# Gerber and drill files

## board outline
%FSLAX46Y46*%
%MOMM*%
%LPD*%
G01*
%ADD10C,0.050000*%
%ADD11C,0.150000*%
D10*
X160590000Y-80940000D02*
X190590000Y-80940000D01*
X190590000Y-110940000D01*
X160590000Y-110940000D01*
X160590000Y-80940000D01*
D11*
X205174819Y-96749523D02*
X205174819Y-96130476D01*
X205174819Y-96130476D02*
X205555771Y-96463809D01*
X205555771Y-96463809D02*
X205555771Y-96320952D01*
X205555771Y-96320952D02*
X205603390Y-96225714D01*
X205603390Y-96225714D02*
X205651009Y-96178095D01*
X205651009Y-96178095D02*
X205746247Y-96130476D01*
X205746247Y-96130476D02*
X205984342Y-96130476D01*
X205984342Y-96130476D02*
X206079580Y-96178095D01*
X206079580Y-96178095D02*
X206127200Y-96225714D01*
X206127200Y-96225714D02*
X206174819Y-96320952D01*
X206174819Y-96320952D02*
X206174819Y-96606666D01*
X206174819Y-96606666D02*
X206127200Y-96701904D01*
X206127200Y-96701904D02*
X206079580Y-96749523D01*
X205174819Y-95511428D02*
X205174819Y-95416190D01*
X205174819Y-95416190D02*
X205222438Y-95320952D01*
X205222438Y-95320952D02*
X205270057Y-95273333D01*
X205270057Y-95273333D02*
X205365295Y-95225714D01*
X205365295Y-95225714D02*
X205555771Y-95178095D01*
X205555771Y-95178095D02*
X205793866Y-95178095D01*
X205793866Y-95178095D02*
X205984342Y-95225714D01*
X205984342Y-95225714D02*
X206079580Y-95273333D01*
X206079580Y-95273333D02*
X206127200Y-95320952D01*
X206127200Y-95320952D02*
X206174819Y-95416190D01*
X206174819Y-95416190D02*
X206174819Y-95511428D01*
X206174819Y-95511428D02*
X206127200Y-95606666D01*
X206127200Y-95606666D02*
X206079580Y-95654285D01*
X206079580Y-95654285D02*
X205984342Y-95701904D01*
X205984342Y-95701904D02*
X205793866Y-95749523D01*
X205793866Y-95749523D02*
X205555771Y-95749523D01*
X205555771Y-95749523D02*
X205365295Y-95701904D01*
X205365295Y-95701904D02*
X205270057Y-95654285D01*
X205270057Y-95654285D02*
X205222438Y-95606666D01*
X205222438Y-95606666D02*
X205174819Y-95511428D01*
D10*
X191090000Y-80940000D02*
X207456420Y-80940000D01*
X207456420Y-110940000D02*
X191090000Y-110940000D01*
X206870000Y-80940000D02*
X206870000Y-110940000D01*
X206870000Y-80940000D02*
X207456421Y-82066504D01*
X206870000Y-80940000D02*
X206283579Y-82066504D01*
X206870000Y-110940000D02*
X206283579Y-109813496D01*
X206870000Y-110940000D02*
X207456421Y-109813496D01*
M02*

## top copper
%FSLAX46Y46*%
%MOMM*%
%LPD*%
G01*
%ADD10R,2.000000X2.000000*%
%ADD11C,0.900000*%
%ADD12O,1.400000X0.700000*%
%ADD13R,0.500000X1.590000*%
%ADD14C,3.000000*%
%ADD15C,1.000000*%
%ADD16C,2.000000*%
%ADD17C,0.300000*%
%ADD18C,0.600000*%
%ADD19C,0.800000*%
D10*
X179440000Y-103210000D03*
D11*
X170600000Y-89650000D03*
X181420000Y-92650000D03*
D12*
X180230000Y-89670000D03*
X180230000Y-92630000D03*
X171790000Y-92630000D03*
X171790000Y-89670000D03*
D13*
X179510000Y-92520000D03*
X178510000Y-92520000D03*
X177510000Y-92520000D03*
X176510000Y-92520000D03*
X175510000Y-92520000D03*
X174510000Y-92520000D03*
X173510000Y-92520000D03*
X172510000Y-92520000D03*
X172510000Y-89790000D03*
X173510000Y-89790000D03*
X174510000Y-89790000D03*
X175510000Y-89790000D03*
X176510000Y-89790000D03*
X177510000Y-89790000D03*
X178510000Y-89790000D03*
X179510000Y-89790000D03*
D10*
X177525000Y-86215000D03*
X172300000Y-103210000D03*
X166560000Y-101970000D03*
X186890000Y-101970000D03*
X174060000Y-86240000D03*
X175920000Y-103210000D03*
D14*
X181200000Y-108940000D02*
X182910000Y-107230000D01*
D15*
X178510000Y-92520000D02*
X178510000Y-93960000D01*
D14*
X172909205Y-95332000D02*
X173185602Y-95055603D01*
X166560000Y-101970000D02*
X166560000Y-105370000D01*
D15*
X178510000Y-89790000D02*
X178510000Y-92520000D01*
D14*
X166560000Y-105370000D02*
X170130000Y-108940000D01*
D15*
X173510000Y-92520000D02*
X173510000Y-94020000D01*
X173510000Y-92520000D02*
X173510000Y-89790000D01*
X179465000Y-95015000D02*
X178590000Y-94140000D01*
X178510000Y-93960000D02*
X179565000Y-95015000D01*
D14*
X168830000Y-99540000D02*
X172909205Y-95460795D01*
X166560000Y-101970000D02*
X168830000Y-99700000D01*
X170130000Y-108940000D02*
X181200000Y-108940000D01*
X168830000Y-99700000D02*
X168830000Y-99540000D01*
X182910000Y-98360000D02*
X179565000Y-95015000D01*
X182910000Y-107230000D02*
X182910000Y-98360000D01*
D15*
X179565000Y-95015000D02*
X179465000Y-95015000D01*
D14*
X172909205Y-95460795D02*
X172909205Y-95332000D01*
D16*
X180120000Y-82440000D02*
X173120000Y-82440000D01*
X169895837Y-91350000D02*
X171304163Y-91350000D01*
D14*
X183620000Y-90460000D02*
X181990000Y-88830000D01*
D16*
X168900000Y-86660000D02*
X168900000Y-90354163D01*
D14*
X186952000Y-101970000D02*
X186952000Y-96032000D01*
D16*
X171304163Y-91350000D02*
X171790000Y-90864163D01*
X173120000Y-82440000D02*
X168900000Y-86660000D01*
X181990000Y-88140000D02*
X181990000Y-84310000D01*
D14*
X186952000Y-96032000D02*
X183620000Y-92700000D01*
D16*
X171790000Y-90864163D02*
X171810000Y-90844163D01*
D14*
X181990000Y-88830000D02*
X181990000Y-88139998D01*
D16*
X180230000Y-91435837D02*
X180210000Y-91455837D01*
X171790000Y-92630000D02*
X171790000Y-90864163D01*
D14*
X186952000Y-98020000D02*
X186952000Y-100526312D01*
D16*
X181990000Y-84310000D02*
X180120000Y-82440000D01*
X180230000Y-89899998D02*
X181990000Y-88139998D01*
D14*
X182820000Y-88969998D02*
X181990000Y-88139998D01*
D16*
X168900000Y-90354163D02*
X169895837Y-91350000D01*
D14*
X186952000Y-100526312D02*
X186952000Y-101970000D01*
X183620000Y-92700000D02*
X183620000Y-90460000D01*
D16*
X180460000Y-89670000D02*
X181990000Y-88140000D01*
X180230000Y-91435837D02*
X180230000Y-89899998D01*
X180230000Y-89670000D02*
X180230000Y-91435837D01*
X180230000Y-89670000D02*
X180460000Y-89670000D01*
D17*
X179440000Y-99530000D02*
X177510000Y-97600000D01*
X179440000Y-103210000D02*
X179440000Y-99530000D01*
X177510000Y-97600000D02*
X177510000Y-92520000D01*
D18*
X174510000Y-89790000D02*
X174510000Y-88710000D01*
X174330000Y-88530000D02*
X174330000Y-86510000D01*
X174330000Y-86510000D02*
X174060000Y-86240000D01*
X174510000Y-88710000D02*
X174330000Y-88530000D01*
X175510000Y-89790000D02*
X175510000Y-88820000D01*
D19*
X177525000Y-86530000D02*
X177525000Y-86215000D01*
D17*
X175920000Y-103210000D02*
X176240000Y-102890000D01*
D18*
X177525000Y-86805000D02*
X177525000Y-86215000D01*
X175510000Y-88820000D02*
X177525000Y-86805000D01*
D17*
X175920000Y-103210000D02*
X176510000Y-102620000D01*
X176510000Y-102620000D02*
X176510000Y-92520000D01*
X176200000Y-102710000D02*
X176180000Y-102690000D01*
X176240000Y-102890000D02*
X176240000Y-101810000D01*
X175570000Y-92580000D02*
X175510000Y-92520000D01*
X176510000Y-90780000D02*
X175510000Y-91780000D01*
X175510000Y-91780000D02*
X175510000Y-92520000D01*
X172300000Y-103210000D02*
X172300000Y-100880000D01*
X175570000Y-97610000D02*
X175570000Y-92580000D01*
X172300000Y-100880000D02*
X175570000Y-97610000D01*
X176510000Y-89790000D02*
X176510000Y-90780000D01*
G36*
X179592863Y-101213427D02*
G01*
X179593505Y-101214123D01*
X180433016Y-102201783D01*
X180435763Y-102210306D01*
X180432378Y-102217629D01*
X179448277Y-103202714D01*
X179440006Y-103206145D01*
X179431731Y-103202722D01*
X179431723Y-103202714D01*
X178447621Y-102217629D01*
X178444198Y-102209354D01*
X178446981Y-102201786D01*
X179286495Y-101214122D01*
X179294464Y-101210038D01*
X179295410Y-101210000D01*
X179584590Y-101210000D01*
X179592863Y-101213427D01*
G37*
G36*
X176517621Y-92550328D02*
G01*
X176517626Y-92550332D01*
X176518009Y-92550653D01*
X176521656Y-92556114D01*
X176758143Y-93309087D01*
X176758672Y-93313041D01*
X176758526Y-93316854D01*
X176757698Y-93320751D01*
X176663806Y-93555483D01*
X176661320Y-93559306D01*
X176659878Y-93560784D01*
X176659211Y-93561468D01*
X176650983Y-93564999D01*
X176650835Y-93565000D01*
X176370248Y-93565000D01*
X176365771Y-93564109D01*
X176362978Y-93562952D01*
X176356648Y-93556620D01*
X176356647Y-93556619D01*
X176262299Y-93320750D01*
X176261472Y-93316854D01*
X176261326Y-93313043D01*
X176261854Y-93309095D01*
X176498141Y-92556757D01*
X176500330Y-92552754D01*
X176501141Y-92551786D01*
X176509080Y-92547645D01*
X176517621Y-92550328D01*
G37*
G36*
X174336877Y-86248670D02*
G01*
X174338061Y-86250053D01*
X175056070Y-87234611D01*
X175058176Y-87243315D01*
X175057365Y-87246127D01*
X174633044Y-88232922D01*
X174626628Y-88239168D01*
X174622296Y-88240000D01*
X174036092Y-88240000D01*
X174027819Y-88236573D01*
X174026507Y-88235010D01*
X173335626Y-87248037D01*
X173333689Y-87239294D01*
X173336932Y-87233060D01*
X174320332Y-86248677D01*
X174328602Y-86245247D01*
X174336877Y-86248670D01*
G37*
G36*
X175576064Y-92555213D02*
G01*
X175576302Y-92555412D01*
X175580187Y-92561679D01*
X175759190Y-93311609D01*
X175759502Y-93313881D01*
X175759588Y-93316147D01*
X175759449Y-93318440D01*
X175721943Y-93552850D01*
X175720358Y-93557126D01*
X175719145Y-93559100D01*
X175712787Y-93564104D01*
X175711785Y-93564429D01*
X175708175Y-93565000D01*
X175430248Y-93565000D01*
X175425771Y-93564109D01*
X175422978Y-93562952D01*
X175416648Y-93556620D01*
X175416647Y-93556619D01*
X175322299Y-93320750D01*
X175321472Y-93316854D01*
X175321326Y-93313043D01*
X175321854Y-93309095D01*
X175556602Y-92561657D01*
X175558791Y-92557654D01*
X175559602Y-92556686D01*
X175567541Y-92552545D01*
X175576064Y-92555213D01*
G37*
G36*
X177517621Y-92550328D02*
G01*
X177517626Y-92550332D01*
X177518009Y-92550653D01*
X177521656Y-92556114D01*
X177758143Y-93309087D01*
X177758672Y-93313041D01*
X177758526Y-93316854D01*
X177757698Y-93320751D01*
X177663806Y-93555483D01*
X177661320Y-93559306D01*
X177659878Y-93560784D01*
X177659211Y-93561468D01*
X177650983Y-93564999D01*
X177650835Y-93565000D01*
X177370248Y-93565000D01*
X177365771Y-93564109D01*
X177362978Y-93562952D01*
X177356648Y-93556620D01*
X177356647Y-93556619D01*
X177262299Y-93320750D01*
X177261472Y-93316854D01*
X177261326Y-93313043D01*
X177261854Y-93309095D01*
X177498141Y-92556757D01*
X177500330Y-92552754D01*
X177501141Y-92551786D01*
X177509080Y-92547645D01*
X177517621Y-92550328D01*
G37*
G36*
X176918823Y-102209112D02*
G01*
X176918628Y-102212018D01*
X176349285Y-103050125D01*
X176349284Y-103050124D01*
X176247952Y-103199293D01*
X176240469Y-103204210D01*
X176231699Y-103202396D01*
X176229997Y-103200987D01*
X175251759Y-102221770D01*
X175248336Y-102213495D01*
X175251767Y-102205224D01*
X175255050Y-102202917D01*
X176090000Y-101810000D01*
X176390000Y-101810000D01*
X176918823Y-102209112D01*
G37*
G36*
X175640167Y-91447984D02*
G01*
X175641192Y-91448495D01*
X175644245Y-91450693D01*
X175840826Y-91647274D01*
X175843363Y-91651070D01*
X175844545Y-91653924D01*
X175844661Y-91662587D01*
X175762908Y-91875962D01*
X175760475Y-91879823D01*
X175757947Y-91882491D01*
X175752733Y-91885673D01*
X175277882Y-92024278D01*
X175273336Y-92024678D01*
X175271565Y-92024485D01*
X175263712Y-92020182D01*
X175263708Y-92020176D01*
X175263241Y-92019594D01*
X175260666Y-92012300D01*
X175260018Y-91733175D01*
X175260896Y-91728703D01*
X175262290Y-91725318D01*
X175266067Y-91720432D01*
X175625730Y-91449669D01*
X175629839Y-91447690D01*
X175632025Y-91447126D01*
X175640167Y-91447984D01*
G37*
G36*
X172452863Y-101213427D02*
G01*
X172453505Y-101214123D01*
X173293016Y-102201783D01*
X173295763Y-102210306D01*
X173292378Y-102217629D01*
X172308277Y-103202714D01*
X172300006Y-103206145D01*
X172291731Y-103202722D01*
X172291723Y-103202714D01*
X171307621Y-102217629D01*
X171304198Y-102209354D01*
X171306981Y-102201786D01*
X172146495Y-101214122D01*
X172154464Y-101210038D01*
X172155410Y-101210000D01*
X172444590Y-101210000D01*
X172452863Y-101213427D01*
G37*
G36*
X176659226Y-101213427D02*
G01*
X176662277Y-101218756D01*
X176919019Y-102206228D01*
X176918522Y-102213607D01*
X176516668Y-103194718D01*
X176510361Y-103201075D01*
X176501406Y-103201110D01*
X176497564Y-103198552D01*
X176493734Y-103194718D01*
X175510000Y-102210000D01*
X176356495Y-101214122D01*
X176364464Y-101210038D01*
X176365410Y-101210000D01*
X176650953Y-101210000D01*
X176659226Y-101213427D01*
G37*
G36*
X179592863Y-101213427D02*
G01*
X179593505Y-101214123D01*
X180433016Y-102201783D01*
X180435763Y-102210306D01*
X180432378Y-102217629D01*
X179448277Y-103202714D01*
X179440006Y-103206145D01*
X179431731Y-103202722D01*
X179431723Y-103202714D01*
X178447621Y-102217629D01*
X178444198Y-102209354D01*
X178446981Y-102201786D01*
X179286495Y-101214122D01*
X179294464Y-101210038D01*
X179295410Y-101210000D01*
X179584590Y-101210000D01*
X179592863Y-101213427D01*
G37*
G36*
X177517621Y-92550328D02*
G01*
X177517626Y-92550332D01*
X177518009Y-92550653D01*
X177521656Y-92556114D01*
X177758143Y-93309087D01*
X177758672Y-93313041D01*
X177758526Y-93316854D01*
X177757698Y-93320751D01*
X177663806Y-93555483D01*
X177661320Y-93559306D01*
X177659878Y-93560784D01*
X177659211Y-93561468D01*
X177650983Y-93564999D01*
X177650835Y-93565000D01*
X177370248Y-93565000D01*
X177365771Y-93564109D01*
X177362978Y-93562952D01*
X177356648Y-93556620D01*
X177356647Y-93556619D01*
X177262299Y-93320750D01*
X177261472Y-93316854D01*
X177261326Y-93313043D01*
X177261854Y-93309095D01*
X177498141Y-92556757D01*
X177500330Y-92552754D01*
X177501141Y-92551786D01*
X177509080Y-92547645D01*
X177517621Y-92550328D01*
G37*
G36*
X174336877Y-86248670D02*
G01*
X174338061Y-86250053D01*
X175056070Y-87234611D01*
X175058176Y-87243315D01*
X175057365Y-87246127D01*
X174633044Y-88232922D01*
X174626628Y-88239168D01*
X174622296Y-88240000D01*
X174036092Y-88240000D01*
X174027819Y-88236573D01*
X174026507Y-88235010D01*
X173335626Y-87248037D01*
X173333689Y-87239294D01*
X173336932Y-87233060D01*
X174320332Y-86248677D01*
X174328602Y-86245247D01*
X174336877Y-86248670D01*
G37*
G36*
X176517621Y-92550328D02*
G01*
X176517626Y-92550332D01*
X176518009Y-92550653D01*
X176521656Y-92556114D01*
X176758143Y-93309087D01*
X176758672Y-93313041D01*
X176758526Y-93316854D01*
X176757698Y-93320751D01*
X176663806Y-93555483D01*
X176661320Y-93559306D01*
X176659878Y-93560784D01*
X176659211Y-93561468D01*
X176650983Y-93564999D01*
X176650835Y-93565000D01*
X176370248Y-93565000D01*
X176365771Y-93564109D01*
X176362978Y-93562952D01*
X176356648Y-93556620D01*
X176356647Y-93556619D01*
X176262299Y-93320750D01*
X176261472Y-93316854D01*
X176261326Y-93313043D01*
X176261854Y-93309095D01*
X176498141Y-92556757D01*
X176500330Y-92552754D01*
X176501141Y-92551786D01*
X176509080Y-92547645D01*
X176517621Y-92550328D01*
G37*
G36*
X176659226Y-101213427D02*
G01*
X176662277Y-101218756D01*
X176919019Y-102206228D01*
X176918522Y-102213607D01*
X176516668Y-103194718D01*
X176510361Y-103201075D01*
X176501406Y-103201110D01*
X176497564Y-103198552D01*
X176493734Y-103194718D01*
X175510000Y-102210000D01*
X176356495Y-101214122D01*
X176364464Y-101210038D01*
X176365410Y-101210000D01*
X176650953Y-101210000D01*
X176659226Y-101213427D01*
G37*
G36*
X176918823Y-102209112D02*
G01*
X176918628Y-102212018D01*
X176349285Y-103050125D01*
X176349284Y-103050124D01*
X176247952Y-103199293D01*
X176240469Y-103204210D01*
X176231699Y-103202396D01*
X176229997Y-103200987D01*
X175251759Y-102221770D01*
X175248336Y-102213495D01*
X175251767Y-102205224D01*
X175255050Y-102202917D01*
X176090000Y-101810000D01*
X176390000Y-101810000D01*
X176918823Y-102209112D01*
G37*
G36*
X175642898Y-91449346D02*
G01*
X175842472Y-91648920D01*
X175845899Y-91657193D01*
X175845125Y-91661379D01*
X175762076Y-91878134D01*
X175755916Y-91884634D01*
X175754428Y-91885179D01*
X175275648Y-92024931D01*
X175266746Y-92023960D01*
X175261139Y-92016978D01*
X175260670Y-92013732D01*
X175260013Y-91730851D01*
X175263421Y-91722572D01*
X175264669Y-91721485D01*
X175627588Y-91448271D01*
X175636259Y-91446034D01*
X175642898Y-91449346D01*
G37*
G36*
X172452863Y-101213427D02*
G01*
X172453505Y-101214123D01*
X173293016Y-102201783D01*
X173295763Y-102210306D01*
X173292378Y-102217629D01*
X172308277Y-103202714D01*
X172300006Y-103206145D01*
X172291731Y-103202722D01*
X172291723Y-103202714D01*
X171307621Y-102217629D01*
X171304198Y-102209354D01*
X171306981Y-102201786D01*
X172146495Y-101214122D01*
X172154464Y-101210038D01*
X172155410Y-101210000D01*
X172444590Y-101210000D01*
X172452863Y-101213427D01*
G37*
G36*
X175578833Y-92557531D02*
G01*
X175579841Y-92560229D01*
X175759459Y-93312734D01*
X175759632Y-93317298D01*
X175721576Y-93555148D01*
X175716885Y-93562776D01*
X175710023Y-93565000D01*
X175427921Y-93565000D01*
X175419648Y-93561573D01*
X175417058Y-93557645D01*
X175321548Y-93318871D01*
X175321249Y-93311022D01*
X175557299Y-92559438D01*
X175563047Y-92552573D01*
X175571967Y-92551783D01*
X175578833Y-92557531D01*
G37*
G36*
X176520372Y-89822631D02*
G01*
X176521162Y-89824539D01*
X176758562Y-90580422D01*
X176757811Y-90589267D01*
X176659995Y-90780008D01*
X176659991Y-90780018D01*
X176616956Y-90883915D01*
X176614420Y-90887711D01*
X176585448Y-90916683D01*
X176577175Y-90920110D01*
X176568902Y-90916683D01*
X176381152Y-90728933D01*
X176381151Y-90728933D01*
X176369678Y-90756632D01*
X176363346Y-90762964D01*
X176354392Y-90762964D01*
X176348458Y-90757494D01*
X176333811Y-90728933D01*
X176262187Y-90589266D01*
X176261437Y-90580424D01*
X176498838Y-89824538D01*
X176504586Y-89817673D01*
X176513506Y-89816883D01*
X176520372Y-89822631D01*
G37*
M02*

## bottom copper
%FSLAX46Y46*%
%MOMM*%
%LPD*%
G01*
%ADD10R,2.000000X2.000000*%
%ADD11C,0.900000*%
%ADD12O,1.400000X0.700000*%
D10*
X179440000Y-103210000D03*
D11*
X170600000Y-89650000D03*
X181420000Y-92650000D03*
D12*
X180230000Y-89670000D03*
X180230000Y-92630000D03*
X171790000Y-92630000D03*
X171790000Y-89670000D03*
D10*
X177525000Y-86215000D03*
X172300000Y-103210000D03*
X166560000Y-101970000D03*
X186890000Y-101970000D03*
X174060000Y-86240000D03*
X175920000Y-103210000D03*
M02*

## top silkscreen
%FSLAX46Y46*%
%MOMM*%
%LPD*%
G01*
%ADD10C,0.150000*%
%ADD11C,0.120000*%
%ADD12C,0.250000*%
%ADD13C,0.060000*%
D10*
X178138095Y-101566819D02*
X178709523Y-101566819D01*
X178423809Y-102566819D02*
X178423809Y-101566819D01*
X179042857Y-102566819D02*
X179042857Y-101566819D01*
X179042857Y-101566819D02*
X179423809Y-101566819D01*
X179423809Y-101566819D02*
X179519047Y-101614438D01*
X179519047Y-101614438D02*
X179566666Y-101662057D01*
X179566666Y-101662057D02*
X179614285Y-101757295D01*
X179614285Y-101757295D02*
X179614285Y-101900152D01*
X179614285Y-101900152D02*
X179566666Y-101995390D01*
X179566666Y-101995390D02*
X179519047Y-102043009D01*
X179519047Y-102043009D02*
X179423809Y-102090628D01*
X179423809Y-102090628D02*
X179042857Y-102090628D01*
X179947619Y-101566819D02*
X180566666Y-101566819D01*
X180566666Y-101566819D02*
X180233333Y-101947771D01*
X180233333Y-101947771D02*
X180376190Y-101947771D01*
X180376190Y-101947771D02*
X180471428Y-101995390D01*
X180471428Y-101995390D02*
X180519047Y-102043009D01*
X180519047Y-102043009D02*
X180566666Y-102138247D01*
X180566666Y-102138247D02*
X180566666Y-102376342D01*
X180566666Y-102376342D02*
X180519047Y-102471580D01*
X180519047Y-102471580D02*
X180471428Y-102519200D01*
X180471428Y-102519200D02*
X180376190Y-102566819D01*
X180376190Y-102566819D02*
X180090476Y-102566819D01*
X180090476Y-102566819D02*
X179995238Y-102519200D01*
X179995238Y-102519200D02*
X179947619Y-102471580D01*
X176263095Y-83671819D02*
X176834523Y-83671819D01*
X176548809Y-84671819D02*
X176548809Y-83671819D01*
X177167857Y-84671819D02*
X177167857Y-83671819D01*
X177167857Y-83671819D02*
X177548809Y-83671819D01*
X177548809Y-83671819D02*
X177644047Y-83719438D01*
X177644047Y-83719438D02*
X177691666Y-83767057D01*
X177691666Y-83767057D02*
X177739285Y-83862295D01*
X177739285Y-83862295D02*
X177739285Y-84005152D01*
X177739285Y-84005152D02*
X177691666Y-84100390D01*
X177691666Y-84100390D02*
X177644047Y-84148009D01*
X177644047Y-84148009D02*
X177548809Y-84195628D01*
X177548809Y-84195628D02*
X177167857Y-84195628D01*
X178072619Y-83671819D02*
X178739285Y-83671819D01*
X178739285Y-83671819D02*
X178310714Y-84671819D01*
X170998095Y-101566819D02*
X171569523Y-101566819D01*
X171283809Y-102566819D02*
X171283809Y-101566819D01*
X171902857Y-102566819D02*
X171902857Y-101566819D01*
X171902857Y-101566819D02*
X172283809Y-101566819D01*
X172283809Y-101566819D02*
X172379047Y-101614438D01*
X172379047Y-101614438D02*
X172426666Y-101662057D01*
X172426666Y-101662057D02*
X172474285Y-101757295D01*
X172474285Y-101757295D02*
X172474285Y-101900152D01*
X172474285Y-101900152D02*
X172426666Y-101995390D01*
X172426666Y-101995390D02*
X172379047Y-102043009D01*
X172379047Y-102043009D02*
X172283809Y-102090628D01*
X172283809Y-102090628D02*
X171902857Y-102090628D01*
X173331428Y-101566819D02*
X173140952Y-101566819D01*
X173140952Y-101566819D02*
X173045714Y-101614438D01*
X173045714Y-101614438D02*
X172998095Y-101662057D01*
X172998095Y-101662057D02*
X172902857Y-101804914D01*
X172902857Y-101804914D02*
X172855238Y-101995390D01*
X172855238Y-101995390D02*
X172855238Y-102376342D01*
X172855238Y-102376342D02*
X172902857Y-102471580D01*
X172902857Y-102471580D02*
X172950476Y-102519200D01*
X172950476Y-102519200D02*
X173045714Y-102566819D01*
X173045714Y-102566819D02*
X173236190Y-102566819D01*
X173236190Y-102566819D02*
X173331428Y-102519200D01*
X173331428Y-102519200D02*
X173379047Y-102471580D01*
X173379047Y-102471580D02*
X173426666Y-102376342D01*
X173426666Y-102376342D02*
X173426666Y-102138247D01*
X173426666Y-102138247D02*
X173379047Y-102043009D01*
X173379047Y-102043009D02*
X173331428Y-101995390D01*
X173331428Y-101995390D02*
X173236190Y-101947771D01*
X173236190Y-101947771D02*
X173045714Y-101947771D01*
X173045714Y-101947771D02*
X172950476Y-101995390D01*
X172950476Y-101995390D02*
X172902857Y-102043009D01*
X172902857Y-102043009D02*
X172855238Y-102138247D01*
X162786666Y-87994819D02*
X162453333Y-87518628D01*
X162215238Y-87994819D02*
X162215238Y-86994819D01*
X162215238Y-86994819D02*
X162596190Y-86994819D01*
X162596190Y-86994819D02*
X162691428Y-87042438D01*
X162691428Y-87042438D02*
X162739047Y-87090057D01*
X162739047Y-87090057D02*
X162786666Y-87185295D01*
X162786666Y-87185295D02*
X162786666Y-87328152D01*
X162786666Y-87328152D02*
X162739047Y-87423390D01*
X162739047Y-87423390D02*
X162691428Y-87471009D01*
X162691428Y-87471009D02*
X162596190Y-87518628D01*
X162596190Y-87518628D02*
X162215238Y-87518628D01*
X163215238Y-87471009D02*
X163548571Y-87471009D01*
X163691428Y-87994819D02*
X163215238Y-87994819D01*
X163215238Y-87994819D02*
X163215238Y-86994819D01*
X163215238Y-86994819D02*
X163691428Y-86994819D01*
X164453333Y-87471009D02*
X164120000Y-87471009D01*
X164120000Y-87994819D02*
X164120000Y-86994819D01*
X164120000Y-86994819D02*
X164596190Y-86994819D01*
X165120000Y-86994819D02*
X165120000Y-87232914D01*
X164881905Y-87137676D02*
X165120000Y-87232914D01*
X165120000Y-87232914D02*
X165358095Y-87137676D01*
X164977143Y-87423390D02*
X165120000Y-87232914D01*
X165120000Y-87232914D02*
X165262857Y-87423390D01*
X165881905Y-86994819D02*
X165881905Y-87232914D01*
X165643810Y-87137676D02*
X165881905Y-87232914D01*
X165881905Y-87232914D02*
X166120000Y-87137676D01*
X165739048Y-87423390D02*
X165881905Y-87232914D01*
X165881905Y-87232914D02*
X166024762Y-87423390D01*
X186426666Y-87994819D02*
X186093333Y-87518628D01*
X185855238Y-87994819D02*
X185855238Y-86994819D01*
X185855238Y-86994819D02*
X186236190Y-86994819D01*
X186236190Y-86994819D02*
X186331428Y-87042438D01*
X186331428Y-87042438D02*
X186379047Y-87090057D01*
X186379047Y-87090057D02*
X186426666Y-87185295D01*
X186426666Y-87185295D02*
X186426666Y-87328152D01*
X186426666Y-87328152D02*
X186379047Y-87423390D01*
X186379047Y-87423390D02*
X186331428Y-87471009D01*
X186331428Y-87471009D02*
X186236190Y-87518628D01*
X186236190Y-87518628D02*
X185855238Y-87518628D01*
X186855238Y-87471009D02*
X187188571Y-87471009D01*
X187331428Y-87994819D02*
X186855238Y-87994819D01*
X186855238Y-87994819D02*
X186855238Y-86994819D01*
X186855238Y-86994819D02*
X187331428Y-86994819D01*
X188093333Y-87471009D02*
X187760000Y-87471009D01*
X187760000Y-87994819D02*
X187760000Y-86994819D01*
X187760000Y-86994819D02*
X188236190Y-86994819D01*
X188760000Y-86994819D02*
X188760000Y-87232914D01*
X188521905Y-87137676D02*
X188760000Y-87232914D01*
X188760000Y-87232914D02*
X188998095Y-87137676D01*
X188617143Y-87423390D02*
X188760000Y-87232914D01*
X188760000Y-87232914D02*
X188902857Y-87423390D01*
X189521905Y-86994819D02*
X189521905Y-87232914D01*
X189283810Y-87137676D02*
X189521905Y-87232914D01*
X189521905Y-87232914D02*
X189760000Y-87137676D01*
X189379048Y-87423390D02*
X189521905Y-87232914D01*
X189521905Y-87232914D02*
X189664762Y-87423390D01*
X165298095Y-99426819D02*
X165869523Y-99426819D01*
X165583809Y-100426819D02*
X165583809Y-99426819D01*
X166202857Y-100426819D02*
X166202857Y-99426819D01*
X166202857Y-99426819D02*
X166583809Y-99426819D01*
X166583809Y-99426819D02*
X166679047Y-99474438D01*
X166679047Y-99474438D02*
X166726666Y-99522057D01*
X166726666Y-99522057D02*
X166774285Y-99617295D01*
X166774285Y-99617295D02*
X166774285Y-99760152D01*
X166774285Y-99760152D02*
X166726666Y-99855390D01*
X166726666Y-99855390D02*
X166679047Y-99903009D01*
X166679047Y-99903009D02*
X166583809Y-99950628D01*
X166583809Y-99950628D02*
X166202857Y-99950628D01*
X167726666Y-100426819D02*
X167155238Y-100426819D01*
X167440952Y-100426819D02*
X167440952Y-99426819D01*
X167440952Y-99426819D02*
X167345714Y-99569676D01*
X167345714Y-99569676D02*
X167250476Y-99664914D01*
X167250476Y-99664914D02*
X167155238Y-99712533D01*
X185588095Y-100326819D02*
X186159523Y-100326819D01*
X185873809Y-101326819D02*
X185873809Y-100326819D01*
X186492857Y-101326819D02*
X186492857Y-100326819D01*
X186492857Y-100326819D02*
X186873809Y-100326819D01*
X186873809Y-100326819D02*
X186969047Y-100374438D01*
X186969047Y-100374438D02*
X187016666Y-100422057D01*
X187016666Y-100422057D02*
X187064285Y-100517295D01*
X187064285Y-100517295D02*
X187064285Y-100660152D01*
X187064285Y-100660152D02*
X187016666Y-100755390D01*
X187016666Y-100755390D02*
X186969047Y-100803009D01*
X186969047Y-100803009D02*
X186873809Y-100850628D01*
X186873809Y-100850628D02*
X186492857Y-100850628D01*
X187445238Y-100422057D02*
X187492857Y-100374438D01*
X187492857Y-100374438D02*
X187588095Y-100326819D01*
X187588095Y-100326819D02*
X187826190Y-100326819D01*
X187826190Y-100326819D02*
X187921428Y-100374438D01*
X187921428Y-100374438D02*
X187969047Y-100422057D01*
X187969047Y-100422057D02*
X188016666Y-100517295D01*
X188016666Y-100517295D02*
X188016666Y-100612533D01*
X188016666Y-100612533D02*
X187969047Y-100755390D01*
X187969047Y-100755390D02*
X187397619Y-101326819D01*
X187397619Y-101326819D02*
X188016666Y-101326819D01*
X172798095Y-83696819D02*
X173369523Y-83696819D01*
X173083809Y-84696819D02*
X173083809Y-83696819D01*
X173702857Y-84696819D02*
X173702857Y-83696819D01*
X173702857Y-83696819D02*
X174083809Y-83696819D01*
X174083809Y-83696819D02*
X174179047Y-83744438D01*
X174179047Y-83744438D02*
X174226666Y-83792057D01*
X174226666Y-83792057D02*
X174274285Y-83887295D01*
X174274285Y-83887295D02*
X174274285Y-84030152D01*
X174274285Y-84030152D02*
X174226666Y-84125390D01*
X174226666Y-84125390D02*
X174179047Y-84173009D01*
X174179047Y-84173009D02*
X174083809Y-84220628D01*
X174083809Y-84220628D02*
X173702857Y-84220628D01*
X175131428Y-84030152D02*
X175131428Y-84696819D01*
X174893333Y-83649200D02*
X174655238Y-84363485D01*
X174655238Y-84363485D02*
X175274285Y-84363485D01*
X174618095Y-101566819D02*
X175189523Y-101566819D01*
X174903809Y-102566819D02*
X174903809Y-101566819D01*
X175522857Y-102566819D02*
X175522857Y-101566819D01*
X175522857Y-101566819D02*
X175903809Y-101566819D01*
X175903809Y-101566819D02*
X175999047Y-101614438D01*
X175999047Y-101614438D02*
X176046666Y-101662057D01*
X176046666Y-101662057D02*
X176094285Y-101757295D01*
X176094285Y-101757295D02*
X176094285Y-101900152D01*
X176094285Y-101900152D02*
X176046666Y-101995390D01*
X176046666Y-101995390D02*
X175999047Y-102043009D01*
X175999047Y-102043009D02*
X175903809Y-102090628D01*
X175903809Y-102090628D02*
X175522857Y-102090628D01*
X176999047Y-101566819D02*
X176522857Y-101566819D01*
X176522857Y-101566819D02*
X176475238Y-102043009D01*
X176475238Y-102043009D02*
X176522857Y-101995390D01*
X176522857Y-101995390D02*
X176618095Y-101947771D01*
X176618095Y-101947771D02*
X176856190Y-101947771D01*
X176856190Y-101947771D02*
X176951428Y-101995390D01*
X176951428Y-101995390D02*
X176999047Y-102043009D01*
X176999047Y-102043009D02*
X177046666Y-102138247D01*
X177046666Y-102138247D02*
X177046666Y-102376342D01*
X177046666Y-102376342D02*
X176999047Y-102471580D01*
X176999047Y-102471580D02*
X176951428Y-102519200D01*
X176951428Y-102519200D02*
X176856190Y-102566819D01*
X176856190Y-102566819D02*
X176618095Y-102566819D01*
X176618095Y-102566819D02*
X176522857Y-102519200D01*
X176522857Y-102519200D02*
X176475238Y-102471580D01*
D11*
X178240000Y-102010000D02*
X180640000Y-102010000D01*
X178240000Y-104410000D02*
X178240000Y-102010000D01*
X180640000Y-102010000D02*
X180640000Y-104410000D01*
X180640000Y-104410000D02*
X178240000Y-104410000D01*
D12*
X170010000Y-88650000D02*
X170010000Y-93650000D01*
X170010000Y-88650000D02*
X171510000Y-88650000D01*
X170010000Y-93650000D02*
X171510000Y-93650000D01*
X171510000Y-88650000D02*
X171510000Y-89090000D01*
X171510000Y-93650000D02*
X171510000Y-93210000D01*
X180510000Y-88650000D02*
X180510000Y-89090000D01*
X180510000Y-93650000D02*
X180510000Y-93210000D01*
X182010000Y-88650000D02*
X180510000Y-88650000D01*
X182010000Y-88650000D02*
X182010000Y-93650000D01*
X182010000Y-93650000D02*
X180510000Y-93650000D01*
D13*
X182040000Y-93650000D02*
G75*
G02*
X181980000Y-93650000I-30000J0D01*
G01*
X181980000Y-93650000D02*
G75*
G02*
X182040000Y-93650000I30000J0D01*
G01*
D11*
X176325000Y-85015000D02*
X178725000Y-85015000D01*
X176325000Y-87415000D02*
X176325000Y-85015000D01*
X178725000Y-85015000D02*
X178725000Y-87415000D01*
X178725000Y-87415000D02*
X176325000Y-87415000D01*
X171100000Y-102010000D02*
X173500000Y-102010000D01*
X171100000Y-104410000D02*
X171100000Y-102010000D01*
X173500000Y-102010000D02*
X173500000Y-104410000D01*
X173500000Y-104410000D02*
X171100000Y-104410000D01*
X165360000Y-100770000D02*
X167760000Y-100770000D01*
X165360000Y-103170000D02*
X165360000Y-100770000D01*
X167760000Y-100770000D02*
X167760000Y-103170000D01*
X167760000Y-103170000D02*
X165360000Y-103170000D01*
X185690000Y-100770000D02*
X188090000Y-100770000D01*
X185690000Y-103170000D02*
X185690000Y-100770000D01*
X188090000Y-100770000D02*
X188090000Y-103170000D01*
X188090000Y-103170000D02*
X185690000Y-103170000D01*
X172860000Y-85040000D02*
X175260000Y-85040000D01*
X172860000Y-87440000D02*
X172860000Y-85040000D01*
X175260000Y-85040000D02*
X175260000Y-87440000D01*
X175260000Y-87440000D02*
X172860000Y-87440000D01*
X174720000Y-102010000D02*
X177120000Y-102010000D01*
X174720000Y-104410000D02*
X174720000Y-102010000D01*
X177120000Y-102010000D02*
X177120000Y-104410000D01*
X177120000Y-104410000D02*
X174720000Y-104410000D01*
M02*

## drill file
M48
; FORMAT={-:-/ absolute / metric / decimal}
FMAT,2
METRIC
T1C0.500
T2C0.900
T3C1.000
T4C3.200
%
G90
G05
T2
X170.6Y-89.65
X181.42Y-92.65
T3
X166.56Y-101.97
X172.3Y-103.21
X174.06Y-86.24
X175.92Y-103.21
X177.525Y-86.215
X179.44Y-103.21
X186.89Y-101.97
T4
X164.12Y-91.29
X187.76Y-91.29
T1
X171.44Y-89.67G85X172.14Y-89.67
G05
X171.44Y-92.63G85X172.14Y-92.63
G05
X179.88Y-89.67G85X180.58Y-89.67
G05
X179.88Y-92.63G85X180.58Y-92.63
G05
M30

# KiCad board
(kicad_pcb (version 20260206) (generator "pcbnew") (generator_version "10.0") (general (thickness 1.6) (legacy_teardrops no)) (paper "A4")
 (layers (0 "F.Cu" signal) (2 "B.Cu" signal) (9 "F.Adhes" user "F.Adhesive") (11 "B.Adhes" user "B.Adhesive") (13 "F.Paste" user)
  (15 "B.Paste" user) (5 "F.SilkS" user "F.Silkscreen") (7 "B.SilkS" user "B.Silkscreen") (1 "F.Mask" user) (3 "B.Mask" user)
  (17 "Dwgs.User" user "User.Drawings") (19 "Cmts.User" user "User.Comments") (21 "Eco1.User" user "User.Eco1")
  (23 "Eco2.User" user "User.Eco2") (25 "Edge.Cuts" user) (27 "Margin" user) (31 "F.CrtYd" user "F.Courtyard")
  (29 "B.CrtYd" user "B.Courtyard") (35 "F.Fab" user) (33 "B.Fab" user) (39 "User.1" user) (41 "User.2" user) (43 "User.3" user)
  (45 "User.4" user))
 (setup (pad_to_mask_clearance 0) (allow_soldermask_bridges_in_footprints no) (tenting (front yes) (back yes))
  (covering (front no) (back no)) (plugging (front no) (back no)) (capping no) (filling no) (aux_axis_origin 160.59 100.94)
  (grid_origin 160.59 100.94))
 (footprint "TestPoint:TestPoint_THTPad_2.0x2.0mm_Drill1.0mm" (layer "F.Cu") (at 179.44 103.21)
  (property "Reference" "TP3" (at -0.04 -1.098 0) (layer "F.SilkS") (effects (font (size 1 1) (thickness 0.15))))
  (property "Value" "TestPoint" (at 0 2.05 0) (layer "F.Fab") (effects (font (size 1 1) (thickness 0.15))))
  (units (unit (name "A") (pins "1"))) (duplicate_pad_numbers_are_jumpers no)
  (fp_line (start -1.2 -1.2) (end 1.2 -1.2) (stroke (width 0.12) (type solid)) (layer "F.SilkS"))
  (fp_line (start -1.2 1.2) (end -1.2 -1.2) (stroke (width 0.12) (type solid)) (layer "F.SilkS"))
  (fp_line (start 1.2 -1.2) (end 1.2 1.2) (stroke (width 0.12) (type solid)) (layer "F.SilkS"))
  (fp_line (start 1.2 1.2) (end -1.2 1.2) (stroke (width 0.12) (type solid)) (layer "F.SilkS"))
  (pad "1" thru_hole rect (at 0 0) (size 2 2) (drill 1) (layers "*.Cu" "*.Mask") (remove_unused_layers no) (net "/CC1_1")
   (teardrops (best_length_ratio 0.5) (max_length 1) (best_width_ratio 1) (max_width 2) (curved_edges no) (filter_ratio 0.9) (enabled yes)
    (allow_two_segments yes) (prefer_zone_connections yes))))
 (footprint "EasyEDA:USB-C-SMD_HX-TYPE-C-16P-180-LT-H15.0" (layer "F.Cu") (at 176.01 91.15)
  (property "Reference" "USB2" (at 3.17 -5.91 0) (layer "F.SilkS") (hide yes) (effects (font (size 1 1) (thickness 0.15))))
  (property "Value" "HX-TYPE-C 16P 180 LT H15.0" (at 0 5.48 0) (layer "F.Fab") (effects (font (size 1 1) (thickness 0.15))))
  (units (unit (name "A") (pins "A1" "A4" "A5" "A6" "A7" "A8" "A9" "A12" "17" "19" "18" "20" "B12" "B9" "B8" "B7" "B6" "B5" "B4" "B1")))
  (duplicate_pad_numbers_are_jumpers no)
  (fp_line (start -6 -2.5) (end -6 2.5) (stroke (width 0.25) (type solid)) (layer "F.SilkS"))
  (fp_line (start -6 -2.5) (end -4.5 -2.5) (stroke (width 0.25) (type solid)) (layer "F.SilkS"))
  (fp_line (start -6 2.5) (end -4.5 2.5) (stroke (width 0.25) (type solid)) (layer "F.SilkS"))
  (fp_line (start -4.5 -2.5) (end -4.5 -2.06) (stroke (width 0.25) (type solid)) (layer "F.SilkS"))
  (fp_line (start -4.5 2.5) (end -4.5 2.06) (stroke (width 0.25) (type solid)) (layer "F.SilkS"))
  (fp_line (start 4.5 -2.5) (end 4.5 -2.06) (stroke (width 0.25) (type solid)) (layer "F.SilkS"))
  (fp_line (start 4.5 2.5) (end 4.5 2.06) (stroke (width 0.25) (type solid)) (layer "F.SilkS"))
  (fp_line (start 6 -2.5) (end 4.5 -2.5) (stroke (width 0.25) (type solid)) (layer "F.SilkS"))
  (fp_line (start 6 -2.5) (end 6 2.5) (stroke (width 0.25) (type solid)) (layer "F.SilkS"))
  (fp_line (start 6 2.5) (end 4.5 2.5) (stroke (width 0.25) (type solid)) (layer "F.SilkS"))
  (fp_circle (center 6 2.5) (end 6.03 2.5) (stroke (width 0.06) (type solid)) (fill no) (layer "F.SilkS"))
  (pad "" thru_hole circle (at -5.41 -1.5) (size 0.9 0.9) (drill 0.9) (layers "*.Cu" "*.Mask") (remove_unused_layers no)
   (teardrops (best_length_ratio 0.5) (max_length 1) (best_width_ratio 1) (max_width 2) (curved_edges no) (filter_ratio 0.9) (enabled yes)
    (allow_two_segments yes) (prefer_zone_connections yes)))
  (pad "" thru_hole circle (at 5.41 1.5) (size 0.9 0.9) (drill 0.9) (layers "*.Cu" "*.Mask") (remove_unused_layers no)
   (teardrops (best_length_ratio 0.5) (max_length 1) (best_width_ratio 1) (max_width 2) (curved_edges no) (filter_ratio 0.9) (enabled yes)
    (allow_two_segments yes) (prefer_zone_connections yes)))
  (pad "17" thru_hole oval (at 4.22 -1.48 90) (size 0.7 1.4) (drill oval 0.500024 1.199998) (layers "*.Cu" "*.Mask")
   (remove_unused_layers no) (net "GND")
   (teardrops (best_length_ratio 0.5) (max_length 1) (best_width_ratio 1) (max_width 2) (curved_edges no) (filter_ratio 0.9) (enabled yes)
    (allow_two_segments yes) (prefer_zone_connections yes)))
  (pad "18" thru_hole oval (at 4.22 1.48 90) (size 0.7 1.4) (drill oval 0.500024 1.199998) (layers "*.Cu" "*.Mask")
   (remove_unused_layers no) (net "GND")
   (teardrops (best_length_ratio 0.5) (max_length 1) (best_width_ratio 1) (max_width 2) (curved_edges no) (filter_ratio 0.9) (enabled yes)
    (allow_two_segments yes) (prefer_zone_connections yes)))
  (pad "19" thru_hole oval (at -4.22 1.48 90) (size 0.7 1.4) (drill oval 0.500024 1.199998) (layers "*.Cu" "*.Mask")
   (remove_unused_layers no) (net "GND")
   (teardrops (best_length_ratio 0.5) (max_length 1) (best_width_ratio 1) (max_width 2) (curved_edges no) (filter_ratio 0.9) (enabled yes)
    (allow_two_segments yes) (prefer_zone_connections yes)))
  (pad "20" thru_hole oval (at -4.22 -1.48 90) (size 0.7 1.4) (drill oval 0.500024 1.199998) (layers "*.Cu" "*.Mask")
   (remove_unused_layers no) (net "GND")
   (teardrops (best_length_ratio 0.5) (max_length 1) (best_width_ratio 1) (max_width 2) (curved_edges no) (filter_ratio 0.9) (enabled yes)
    (allow_two_segments yes) (prefer_zone_connections yes)))
  (pad "A1" smd rect (at 3.5 1.37) (size 0.5 1.59) (layers "F.Cu" "F.Mask" "F.Paste") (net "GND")
   (teardrops (best_length_ratio 0.5) (max_length 1) (best_width_ratio 1) (max_width 2) (curved_edges no) (filter_ratio 0.9) (enabled yes)
    (allow_two_segments yes) (prefer_zone_connections yes)))
  (pad "A4" smd rect (at 2.5 1.37) (size 0.5 1.59) (layers "F.Cu" "F.Mask" "F.Paste") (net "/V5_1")
   (teardrops (best_length_ratio 0.5) (max_length 1) (best_width_ratio 1) (max_width 2) (curved_edges no) (filter_ratio 0.9) (enabled yes)
    (allow_two_segments yes) (prefer_zone_connections yes)))
  (pad "A5" smd rect (at 1.5 1.37) (size 0.5 1.59) (layers "F.Cu" "F.Mask" "F.Paste") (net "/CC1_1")
   (teardrops (best_length_ratio 0.5) (max_length 1) (best_width_ratio 1) (max_width 2) (curved_edges no) (filter_ratio 0.9) (enabled yes)
    (allow_two_segments yes) (prefer_zone_connections yes)))
  (pad "A6" smd rect (at 0.5 1.37) (size 0.5 1.59) (layers "F.Cu" "F.Mask" "F.Paste") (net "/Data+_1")
   (teardrops (best_length_ratio 0.5) (max_length 1) (best_width_ratio 1) (max_width 2) (curved_edges no) (filter_ratio 0.9) (enabled yes)
    (allow_two_segments yes) (prefer_zone_connections yes)))
  (pad "A7" smd rect (at -0.5 1.37) (size 0.5 1.59) (layers "F.Cu" "F.Mask" "F.Paste") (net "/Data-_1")
   (teardrops (best_length_ratio 0.5) (max_length 1) (best_width_ratio 1) (max_width 2) (curved_edges no) (filter_ratio 0.9) (enabled yes)
    (allow_two_segments yes) (prefer_zone_connections yes)))
  (pad "A8" smd rect (at -1.5 1.37) (size 0.5 1.59) (layers "F.Cu" "F.Mask" "F.Paste") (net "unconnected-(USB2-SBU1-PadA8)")
   (teardrops (best_length_ratio 0.5) (max_length 1) (best_width_ratio 1) (max_width 2) (curved_edges no) (filter_ratio 0.9) (enabled yes)
    (allow_two_segments yes) (prefer_zone_connections yes)))
  (pad "A9" smd rect (at -2.5 1.37) (size 0.5 1.59) (layers "F.Cu" "F.Mask" "F.Paste") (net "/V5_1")
   (teardrops (best_length_ratio 0.5) (max_length 1) (best_width_ratio 1) (max_width 2) (curved_edges no) (filter_ratio 0.9) (enabled yes)
    (allow_two_segments yes) (prefer_zone_connections yes)))
  (pad "A12" smd rect (at -3.5 1.37) (size 0.5 1.59) (layers "F.Cu" "F.Mask" "F.Paste") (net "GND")
   (teardrops (best_length_ratio 0.5) (max_length 1) (best_width_ratio 1) (max_width 2) (curved_edges no) (filter_ratio 0.9) (enabled yes)
    (allow_two_segments yes) (prefer_zone_connections yes)))
  (pad "B1" smd rect (at -3.5 -1.36) (size 0.5 1.59) (layers "F.Cu" "F.Mask" "F.Paste") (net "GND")
   (teardrops (best_length_ratio 0.5) (max_length 1) (best_width_ratio 1) (max_width 2) (curved_edges no) (filter_ratio 0.9) (enabled yes)
    (allow_two_segments yes) (prefer_zone_connections yes)))
  (pad "B4" smd rect (at -2.5 -1.36) (size 0.5 1.59) (layers "F.Cu" "F.Mask" "F.Paste") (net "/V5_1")
   (teardrops (best_length_ratio 0.5) (max_length 1) (best_width_ratio 1) (max_width 2) (curved_edges no) (filter_ratio 0.9) (enabled yes)
    (allow_two_segments yes) (prefer_zone_connections yes)))
  (pad "B5" smd rect (at -1.5 -1.36) (size 0.5 1.59) (layers "F.Cu" "F.Mask" "F.Paste") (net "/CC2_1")
   (teardrops (best_length_ratio 0.5) (max_length 1) (best_width_ratio 1) (max_width 2) (curved_edges no) (filter_ratio 0.9) (enabled yes)
    (allow_two_segments yes) (prefer_zone_connections yes)))
  (pad "B6" smd rect (at -0.5 -1.36) (size 0.5 1.59) (layers "F.Cu" "F.Mask" "F.Paste") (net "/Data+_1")
   (teardrops (best_length_ratio 0.5) (max_length 1) (best_width_ratio 1) (max_width 2) (curved_edges no) (filter_ratio 0.9) (enabled yes)
    (allow_two_segments yes) (prefer_zone_connections yes)))
  (pad "B7" smd rect (at 0.5 -1.36) (size 0.5 1.59) (layers "F.Cu" "F.Mask" "F.Paste") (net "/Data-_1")
   (teardrops (best_length_ratio 0.5) (max_length 1) (best_width_ratio 1) (max_width 2) (curved_edges no) (filter_ratio 0.9) (enabled yes)
    (allow_two_segments yes) (prefer_zone_connections yes)))
  (pad "B8" smd rect (at 1.5 -1.36) (size 0.5 1.59) (layers "F.Cu" "F.Mask" "F.Paste") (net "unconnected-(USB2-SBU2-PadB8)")
   (teardrops (best_length_ratio 0.5) (max_length 1) (best_width_ratio 1) (max_width 2) (curved_edges no) (filter_ratio 0.9) (enabled yes)
    (allow_two_segments yes) (prefer_zone_connections yes)))
  (pad "B9" smd rect (at 2.5 -1.36) (size 0.5 1.59) (layers "F.Cu" "F.Mask" "F.Paste") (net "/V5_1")
   (teardrops (best_length_ratio 0.5) (max_length 1) (best_width_ratio 1) (max_width 2) (curved_edges no) (filter_ratio 0.9) (enabled yes)
    (allow_two_segments yes) (prefer_zone_connections yes)))
  (pad "B12" smd rect (at 3.5 -1.36) (size 0.5 1.59) (layers "F.Cu" "F.Mask" "F.Paste") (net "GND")
   (teardrops (best_length_ratio 0.5) (max_length 1) (best_width_ratio 1) (max_width 2) (curved_edges no) (filter_ratio 0.9) (enabled yes)
    (allow_two_segments yes) (prefer_zone_connections yes))))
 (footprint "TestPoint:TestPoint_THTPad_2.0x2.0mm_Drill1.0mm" (layer "F.Cu") (at 177.525 86.215)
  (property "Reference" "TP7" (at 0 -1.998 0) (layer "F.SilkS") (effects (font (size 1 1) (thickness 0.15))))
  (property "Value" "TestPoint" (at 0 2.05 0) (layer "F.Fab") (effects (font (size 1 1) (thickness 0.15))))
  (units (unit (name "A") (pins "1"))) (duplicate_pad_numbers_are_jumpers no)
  (fp_line (start -1.2 -1.2) (end 1.2 -1.2) (stroke (width 0.12) (type solid)) (layer "F.SilkS"))
  (fp_line (start -1.2 1.2) (end -1.2 -1.2) (stroke (width 0.12) (type solid)) (layer "F.SilkS"))
  (fp_line (start 1.2 -1.2) (end 1.2 1.2) (stroke (width 0.12) (type solid)) (layer "F.SilkS"))
  (fp_line (start 1.2 1.2) (end -1.2 1.2) (stroke (width 0.12) (type solid)) (layer "F.SilkS"))
  (pad "1" thru_hole rect (at 0 0) (size 2 2) (drill 1) (layers "*.Cu" "*.Mask") (remove_unused_layers no) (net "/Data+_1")))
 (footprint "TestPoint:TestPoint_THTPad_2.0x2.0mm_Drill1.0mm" (layer "F.Cu") (at 172.3 103.21)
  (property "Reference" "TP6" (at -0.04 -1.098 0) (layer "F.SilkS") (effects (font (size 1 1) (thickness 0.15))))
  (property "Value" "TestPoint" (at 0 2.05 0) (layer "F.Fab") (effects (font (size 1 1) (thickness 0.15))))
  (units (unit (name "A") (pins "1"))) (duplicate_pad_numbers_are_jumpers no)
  (fp_line (start -1.2 -1.2) (end 1.2 -1.2) (stroke (width 0.12) (type solid)) (layer "F.SilkS"))
  (fp_line (start -1.2 1.2) (end -1.2 -1.2) (stroke (width 0.12) (type solid)) (layer "F.SilkS"))
  (fp_line (start 1.2 -1.2) (end 1.2 1.2) (stroke (width 0.12) (type solid)) (layer "F.SilkS"))
  (fp_line (start 1.2 1.2) (end -1.2 1.2) (stroke (width 0.12) (type solid)) (layer "F.SilkS"))
  (pad "1" thru_hole rect (at 0 0) (size 2 2) (drill 1) (layers "*.Cu" "*.Mask") (remove_unused_layers no) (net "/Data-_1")
   (teardrops (best_length_ratio 0.5) (max_length 1) (best_width_ratio 1) (max_width 2) (curved_edges no) (filter_ratio 0.9) (enabled yes)
    (allow_two_segments yes) (prefer_zone_connections yes))))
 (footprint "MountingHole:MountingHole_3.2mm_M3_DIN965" (layer "F.Cu") (at 164.12 91.29)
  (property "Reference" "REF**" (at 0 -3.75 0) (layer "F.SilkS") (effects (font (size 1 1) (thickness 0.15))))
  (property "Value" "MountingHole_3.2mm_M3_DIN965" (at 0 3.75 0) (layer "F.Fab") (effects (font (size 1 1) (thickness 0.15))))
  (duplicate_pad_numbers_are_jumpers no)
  (pad "" np_thru_hole circle (at 0 0) (size 3.2 3.2) (drill 3.2) (layers "*.Cu" "*.Mask")))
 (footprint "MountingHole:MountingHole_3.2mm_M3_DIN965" (layer "F.Cu") (at 187.76 91.29)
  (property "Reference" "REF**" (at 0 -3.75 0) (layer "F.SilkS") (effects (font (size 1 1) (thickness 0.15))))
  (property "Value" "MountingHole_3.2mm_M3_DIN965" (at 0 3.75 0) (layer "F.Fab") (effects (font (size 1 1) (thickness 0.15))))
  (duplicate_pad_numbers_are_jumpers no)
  (pad "" np_thru_hole circle (at 0 0) (size 3.2 3.2) (drill 3.2) (layers "*.Cu" "*.Mask")))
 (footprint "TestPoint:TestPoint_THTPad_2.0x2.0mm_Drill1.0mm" (layer "F.Cu") (at 166.56 101.97)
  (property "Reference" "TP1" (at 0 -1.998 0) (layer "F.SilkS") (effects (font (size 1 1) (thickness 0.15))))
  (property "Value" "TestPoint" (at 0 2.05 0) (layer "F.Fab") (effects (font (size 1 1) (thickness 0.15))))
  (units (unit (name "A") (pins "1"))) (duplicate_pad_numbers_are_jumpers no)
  (fp_line (start -1.2 -1.2) (end 1.2 -1.2) (stroke (width 0.12) (type solid)) (layer "F.SilkS"))
  (fp_line (start -1.2 1.2) (end -1.2 -1.2) (stroke (width 0.12) (type solid)) (layer "F.SilkS"))
  (fp_line (start 1.2 -1.2) (end 1.2 1.2) (stroke (width 0.12) (type solid)) (layer "F.SilkS"))
  (fp_line (start 1.2 1.2) (end -1.2 1.2) (stroke (width 0.12) (type solid)) (layer "F.SilkS"))
  (pad "1" thru_hole rect (at 0 0) (size 2 2) (drill 1) (layers "*.Cu" "*.Mask") (remove_unused_layers no) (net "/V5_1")
   (teardrops (best_length_ratio 0.5) (max_length 1) (best_width_ratio 1) (max_width 2) (curved_edges no) (filter_ratio 0.9) (enabled yes)
    (allow_two_segments yes) (prefer_zone_connections yes))))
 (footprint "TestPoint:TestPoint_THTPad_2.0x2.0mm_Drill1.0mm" (layer "F.Cu") (at 186.89 101.97)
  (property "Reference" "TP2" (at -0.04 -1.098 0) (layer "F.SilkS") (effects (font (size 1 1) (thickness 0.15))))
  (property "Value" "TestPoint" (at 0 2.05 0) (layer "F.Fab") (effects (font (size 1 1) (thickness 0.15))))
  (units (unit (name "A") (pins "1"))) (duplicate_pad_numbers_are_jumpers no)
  (fp_line (start -1.2 -1.2) (end 1.2 -1.2) (stroke (width 0.12) (type solid)) (layer "F.SilkS"))
  (fp_line (start -1.2 1.2) (end -1.2 -1.2) (stroke (width 0.12) (type solid)) (layer "F.SilkS"))
  (fp_line (start 1.2 -1.2) (end 1.2 1.2) (stroke (width 0.12) (type solid)) (layer "F.SilkS"))
  (fp_line (start 1.2 1.2) (end -1.2 1.2) (stroke (width 0.12) (type solid)) (layer "F.SilkS"))
  (pad "1" thru_hole rect (at 0 0) (size 2 2) (drill 1) (layers "*.Cu" "*.Mask") (remove_unused_layers no) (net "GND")
   (teardrops (best_length_ratio 0.5) (max_length 1) (best_width_ratio 1) (max_width 2) (curved_edges no) (filter_ratio 0.9) (enabled yes)
    (allow_two_segments yes) (prefer_zone_connections yes))))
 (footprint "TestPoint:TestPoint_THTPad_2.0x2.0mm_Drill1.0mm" (layer "F.Cu") (at 174.06 86.24)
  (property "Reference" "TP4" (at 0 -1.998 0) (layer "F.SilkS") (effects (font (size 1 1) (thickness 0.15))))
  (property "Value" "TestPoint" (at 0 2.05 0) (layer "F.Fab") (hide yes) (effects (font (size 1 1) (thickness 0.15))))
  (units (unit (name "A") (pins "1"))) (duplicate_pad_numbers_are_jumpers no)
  (fp_line (start -1.2 -1.2) (end 1.2 -1.2) (stroke (width 0.12) (type solid)) (layer "F.SilkS"))
  (fp_line (start -1.2 1.2) (end -1.2 -1.2) (stroke (width 0.12) (type solid)) (layer "F.SilkS"))
  (fp_line (start 1.2 -1.2) (end 1.2 1.2) (stroke (width 0.12) (type solid)) (layer "F.SilkS"))
  (fp_line (start 1.2 1.2) (end -1.2 1.2) (stroke (width 0.12) (type solid)) (layer "F.SilkS"))
  (pad "1" thru_hole rect (at 0 0) (size 2 2) (drill 1) (layers "*.Cu" "*.Mask") (remove_unused_layers no) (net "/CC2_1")
   (teardrops (best_length_ratio 0.5) (max_length 1) (best_width_ratio 1) (max_width 2) (curved_edges no) (filter_ratio 0.9) (enabled yes)
    (allow_two_segments yes) (prefer_zone_connections yes))))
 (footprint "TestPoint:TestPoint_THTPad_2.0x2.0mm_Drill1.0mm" (layer "F.Cu") (at 175.92 103.21)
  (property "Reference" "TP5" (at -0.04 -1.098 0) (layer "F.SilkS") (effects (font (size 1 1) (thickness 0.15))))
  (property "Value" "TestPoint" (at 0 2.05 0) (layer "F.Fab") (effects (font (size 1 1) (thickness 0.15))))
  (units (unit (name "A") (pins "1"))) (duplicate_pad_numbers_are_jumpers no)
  (fp_line (start -1.2 -1.2) (end 1.2 -1.2) (stroke (width 0.12) (type solid)) (layer "F.SilkS"))
  (fp_line (start -1.2 1.2) (end -1.2 -1.2) (stroke (width 0.12) (type solid)) (layer "F.SilkS"))
  (fp_line (start 1.2 -1.2) (end 1.2 1.2) (stroke (width 0.12) (type solid)) (layer "F.SilkS"))
  (fp_line (start 1.2 1.2) (end -1.2 1.2) (stroke (width 0.12) (type solid)) (layer "F.SilkS"))
  (pad "1" thru_hole rect (at 0 0) (size 2 2) (drill 1) (layers "*.Cu" "*.Mask") (remove_unused_layers no) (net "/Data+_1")
   (teardrops (best_length_ratio 0.5) (max_length 1) (best_width_ratio 1) (max_width 2) (curved_edges no) (filter_ratio 0.9) (enabled yes)
    (allow_two_segments yes) (prefer_zone_connections yes))))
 (gr_rect (start 160.59 80.94) (end 190.59 110.94) (stroke (width 0.05) (type solid)) (fill no) (layer "Edge.Cuts"))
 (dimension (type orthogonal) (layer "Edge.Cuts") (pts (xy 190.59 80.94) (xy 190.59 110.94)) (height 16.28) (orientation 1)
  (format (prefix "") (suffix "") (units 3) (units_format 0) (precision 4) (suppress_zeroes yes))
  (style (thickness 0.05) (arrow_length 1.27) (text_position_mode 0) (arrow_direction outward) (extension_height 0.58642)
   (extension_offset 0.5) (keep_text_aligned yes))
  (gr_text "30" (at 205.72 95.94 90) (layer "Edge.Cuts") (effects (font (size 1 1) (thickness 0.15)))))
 (segment (start 181.2 108.94) (end 182.91 107.23) (width 3) (layer "F.Cu") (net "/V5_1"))
 (segment (start 178.51 92.52) (end 178.51 93.96) (width 1) (layer "F.Cu") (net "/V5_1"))
 (segment (start 172.909205 95.332) (end 173.185602 95.055603) (width 3) (layer "F.Cu") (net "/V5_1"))
 (segment (start 166.56 101.97) (end 166.56 105.37) (width 3) (layer "F.Cu") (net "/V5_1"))
 (segment (start 178.51 89.79) (end 178.51 92.52) (width 1) (layer "F.Cu") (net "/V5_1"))
 (segment (start 166.56 105.37) (end 170.13 108.94) (width 3) (layer "F.Cu") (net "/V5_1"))
 (segment (start 173.51 92.52) (end 173.51 94.02) (width 1) (layer "F.Cu") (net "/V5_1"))
 (segment (start 173.51 92.52) (end 173.51 89.79) (width 1) (layer "F.Cu") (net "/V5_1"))
 (segment (start 179.465 95.015) (end 178.59 94.14) (width 1) (layer "F.Cu") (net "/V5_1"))
 (segment (start 178.51 93.96) (end 179.565 95.015) (width 1) (layer "F.Cu") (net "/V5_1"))
 (segment (start 168.83 99.54) (end 172.909205 95.460795) (width 3) (layer "F.Cu") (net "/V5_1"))
 (segment (start 166.56 101.97) (end 168.83 99.7) (width 3) (layer "F.Cu") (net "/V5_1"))
 (segment (start 170.13 108.94) (end 181.2 108.94) (width 3) (layer "F.Cu") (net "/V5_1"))
 (segment (start 168.83 99.7) (end 168.83 99.54) (width 3) (layer "F.Cu") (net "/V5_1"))
 (segment (start 182.91 98.36) (end 179.565 95.015) (width 3) (layer "F.Cu") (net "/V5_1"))
 (segment (start 182.91 107.23) (end 182.91 98.36) (width 3) (layer "F.Cu") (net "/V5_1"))
 (segment (start 179.565 95.015) (end 179.465 95.015) (width 1) (layer "F.Cu") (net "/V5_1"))
 (segment (start 172.909205 95.460795) (end 172.909205 95.332) (width 3) (layer "F.Cu") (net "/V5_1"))
 (segment (start 180.12 82.44) (end 173.12 82.44) (width 2) (layer "F.Cu") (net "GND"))
 (segment (start 169.895837 91.35) (end 171.304163 91.35) (width 2) (layer "F.Cu") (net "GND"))
 (segment (start 183.62 90.46) (end 181.99 88.83) (width 3) (layer "F.Cu") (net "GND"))
 (segment (start 168.9 86.66) (end 168.9 90.354163) (width 2) (layer "F.Cu") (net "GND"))
 (segment (start 186.952 101.97) (end 186.952 96.032) (width 3) (layer "F.Cu") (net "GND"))
 (segment (start 171.304163 91.35) (end 171.79 90.864163) (width 2) (layer "F.Cu") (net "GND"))
 (segment (start 173.12 82.44) (end 168.9 86.66) (width 2) (layer "F.Cu") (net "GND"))
 (segment (start 181.99 88.14) (end 181.99 84.31) (width 2) (layer "F.Cu") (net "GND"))
 (segment (start 186.952 96.032) (end 183.62 92.7) (width 3) (layer "F.Cu") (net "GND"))
 (segment (start 171.79 90.864163) (end 171.81 90.844163) (width 2) (layer "F.Cu") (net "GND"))
 (segment (start 181.99 88.83) (end 181.99 88.139998) (width 3) (layer "F.Cu") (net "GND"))
 (segment (start 180.23 91.435837) (end 180.21 91.455837) (width 2) (layer "F.Cu") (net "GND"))
 (segment (start 171.79 92.63) (end 171.79 90.864163) (width 2) (layer "F.Cu") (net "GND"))
 (segment (start 186.952 98.02) (end 186.952 100.526312) (width 3) (layer "F.Cu") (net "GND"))
 (segment (start 181.99 84.31) (end 180.12 82.44) (width 2) (layer "F.Cu") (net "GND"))
 (segment (start 180.23 89.899998) (end 181.99 88.139998) (width 2) (layer "F.Cu") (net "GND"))
 (segment (start 182.82 88.969998) (end 181.99 88.139998) (width 3) (layer "F.Cu") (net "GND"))
 (segment (start 168.9 90.354163) (end 169.895837 91.35) (width 2) (layer "F.Cu") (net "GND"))
 (segment (start 186.952 100.526312) (end 186.952 101.97) (width 3) (layer "F.Cu") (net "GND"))
 (segment (start 183.62 92.7) (end 183.62 90.46) (width 3) (layer "F.Cu") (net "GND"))
 (segment (start 180.46 89.67) (end 181.99 88.14) (width 2) (layer "F.Cu") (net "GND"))
 (segment (start 180.23 91.435837) (end 180.23 89.899998) (width 2) (layer "F.Cu") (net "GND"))
 (segment (start 180.23 89.67) (end 180.23 91.435837) (width 2) (layer "F.Cu") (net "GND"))
 (segment (start 180.23 89.67) (end 180.46 89.67) (width 2) (layer "F.Cu") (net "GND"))
 (segment (start 179.44 99.53) (end 177.51 97.6) (width 0.3) (layer "F.Cu") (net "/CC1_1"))
 (segment (start 179.44 103.21) (end 179.44 99.53) (width 0.3) (layer "F.Cu") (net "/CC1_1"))
 (segment (start 177.51 97.6) (end 177.51 92.52) (width 0.3) (layer "F.Cu") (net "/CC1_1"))
 (segment (start 174.51 89.79) (end 174.51 88.71) (width 0.6) (layer "F.Cu") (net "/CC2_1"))
 (segment (start 174.33 88.53) (end 174.33 86.51) (width 0.6) (layer "F.Cu") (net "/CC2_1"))
 (segment (start 174.33 86.51) (end 174.06 86.24) (width 0.6) (layer "F.Cu") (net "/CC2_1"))
 (segment (start 174.51 88.71) (end 174.33 88.53) (width 0.6) (layer "F.Cu") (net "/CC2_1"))
 (segment (start 175.51 89.79) (end 175.51 88.82) (width 0.6) (layer "F.Cu") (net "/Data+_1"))
 (segment (start 177.525 86.53) (end 177.525 86.215) (width 0.8) (layer "F.Cu") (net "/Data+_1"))
 (segment (start 175.92 103.21) (end 176.24 102.89) (width 0.3) (layer "F.Cu") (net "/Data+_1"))
 (segment (start 177.525 86.805) (end 177.525 86.215) (width 0.6) (layer "F.Cu") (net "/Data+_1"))
 (segment (start 175.51 88.82) (end 177.525 86.805) (width 0.6) (layer "F.Cu") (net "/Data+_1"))
 (segment (start 175.92 103.21) (end 176.51 102.62) (width 0.3) (layer "F.Cu") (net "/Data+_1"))
 (segment (start 176.51 102.62) (end 176.51 92.52) (width 0.3) (layer "F.Cu") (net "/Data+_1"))
 (segment (start 176.2 102.71) (end 176.18 102.69) (width 0.3) (layer "F.Cu") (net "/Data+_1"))
 (segment (start 176.24 102.89) (end 176.24 101.81) (width 0.3) (layer "F.Cu") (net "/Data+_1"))
 (segment (start 175.57 92.58) (end 175.51 92.52) (width 0.3) (layer "F.Cu") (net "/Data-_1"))
 (segment (start 176.51 90.78) (end 175.51 91.78) (width 0.3) (layer "F.Cu") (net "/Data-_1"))
 (segment (start 175.51 91.78) (end 175.51 92.52) (width 0.3) (layer "F.Cu") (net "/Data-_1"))
 (segment (start 172.3 103.21) (end 172.3 100.88) (width 0.3) (layer "F.Cu") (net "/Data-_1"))
 (segment (start 175.57 97.61) (end 175.57 92.58) (width 0.3) (layer "F.Cu") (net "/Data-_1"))
 (segment (start 172.3 100.88) (end 175.57 97.61) (width 0.3) (layer "F.Cu") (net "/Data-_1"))
 (segment (start 176.51 89.79) (end 176.51 90.78) (width 0.3) (layer "F.Cu") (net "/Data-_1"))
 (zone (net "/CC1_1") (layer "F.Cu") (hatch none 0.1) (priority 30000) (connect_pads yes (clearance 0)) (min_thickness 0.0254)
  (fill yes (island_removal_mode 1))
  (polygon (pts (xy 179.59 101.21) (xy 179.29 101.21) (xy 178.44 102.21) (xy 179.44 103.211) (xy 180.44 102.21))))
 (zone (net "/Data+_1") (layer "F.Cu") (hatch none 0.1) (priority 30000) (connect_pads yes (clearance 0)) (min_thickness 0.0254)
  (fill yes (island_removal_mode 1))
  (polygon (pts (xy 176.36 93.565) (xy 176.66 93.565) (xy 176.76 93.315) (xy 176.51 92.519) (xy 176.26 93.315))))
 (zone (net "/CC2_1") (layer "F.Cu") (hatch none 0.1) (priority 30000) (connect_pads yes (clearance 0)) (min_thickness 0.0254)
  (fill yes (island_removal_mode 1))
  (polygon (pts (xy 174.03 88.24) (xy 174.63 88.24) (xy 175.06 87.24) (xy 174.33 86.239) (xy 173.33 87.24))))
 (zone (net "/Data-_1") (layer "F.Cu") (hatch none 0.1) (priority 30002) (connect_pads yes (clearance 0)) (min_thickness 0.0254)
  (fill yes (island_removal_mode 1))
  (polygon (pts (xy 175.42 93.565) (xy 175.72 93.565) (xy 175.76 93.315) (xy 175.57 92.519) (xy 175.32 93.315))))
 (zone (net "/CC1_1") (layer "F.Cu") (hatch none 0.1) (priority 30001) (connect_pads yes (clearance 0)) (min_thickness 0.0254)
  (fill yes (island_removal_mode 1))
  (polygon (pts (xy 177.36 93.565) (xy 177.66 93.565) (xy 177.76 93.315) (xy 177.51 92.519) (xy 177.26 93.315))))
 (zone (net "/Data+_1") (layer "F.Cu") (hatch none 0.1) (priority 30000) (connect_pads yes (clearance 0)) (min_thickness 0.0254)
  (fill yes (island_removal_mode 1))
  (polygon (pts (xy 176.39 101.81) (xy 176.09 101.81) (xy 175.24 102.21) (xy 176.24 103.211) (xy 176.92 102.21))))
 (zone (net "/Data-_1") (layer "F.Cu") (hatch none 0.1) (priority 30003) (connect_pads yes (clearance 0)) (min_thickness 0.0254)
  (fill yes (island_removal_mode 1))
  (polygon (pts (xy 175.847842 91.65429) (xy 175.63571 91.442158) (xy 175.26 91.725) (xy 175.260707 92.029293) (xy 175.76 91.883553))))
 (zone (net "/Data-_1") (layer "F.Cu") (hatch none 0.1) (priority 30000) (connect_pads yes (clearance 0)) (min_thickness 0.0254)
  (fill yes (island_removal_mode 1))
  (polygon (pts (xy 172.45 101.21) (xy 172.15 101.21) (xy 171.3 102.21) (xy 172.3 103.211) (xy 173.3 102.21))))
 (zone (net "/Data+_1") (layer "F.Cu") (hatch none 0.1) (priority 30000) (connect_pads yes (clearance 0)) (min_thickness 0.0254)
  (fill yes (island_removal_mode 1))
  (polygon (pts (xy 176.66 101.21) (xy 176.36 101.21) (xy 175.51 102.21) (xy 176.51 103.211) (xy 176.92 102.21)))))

